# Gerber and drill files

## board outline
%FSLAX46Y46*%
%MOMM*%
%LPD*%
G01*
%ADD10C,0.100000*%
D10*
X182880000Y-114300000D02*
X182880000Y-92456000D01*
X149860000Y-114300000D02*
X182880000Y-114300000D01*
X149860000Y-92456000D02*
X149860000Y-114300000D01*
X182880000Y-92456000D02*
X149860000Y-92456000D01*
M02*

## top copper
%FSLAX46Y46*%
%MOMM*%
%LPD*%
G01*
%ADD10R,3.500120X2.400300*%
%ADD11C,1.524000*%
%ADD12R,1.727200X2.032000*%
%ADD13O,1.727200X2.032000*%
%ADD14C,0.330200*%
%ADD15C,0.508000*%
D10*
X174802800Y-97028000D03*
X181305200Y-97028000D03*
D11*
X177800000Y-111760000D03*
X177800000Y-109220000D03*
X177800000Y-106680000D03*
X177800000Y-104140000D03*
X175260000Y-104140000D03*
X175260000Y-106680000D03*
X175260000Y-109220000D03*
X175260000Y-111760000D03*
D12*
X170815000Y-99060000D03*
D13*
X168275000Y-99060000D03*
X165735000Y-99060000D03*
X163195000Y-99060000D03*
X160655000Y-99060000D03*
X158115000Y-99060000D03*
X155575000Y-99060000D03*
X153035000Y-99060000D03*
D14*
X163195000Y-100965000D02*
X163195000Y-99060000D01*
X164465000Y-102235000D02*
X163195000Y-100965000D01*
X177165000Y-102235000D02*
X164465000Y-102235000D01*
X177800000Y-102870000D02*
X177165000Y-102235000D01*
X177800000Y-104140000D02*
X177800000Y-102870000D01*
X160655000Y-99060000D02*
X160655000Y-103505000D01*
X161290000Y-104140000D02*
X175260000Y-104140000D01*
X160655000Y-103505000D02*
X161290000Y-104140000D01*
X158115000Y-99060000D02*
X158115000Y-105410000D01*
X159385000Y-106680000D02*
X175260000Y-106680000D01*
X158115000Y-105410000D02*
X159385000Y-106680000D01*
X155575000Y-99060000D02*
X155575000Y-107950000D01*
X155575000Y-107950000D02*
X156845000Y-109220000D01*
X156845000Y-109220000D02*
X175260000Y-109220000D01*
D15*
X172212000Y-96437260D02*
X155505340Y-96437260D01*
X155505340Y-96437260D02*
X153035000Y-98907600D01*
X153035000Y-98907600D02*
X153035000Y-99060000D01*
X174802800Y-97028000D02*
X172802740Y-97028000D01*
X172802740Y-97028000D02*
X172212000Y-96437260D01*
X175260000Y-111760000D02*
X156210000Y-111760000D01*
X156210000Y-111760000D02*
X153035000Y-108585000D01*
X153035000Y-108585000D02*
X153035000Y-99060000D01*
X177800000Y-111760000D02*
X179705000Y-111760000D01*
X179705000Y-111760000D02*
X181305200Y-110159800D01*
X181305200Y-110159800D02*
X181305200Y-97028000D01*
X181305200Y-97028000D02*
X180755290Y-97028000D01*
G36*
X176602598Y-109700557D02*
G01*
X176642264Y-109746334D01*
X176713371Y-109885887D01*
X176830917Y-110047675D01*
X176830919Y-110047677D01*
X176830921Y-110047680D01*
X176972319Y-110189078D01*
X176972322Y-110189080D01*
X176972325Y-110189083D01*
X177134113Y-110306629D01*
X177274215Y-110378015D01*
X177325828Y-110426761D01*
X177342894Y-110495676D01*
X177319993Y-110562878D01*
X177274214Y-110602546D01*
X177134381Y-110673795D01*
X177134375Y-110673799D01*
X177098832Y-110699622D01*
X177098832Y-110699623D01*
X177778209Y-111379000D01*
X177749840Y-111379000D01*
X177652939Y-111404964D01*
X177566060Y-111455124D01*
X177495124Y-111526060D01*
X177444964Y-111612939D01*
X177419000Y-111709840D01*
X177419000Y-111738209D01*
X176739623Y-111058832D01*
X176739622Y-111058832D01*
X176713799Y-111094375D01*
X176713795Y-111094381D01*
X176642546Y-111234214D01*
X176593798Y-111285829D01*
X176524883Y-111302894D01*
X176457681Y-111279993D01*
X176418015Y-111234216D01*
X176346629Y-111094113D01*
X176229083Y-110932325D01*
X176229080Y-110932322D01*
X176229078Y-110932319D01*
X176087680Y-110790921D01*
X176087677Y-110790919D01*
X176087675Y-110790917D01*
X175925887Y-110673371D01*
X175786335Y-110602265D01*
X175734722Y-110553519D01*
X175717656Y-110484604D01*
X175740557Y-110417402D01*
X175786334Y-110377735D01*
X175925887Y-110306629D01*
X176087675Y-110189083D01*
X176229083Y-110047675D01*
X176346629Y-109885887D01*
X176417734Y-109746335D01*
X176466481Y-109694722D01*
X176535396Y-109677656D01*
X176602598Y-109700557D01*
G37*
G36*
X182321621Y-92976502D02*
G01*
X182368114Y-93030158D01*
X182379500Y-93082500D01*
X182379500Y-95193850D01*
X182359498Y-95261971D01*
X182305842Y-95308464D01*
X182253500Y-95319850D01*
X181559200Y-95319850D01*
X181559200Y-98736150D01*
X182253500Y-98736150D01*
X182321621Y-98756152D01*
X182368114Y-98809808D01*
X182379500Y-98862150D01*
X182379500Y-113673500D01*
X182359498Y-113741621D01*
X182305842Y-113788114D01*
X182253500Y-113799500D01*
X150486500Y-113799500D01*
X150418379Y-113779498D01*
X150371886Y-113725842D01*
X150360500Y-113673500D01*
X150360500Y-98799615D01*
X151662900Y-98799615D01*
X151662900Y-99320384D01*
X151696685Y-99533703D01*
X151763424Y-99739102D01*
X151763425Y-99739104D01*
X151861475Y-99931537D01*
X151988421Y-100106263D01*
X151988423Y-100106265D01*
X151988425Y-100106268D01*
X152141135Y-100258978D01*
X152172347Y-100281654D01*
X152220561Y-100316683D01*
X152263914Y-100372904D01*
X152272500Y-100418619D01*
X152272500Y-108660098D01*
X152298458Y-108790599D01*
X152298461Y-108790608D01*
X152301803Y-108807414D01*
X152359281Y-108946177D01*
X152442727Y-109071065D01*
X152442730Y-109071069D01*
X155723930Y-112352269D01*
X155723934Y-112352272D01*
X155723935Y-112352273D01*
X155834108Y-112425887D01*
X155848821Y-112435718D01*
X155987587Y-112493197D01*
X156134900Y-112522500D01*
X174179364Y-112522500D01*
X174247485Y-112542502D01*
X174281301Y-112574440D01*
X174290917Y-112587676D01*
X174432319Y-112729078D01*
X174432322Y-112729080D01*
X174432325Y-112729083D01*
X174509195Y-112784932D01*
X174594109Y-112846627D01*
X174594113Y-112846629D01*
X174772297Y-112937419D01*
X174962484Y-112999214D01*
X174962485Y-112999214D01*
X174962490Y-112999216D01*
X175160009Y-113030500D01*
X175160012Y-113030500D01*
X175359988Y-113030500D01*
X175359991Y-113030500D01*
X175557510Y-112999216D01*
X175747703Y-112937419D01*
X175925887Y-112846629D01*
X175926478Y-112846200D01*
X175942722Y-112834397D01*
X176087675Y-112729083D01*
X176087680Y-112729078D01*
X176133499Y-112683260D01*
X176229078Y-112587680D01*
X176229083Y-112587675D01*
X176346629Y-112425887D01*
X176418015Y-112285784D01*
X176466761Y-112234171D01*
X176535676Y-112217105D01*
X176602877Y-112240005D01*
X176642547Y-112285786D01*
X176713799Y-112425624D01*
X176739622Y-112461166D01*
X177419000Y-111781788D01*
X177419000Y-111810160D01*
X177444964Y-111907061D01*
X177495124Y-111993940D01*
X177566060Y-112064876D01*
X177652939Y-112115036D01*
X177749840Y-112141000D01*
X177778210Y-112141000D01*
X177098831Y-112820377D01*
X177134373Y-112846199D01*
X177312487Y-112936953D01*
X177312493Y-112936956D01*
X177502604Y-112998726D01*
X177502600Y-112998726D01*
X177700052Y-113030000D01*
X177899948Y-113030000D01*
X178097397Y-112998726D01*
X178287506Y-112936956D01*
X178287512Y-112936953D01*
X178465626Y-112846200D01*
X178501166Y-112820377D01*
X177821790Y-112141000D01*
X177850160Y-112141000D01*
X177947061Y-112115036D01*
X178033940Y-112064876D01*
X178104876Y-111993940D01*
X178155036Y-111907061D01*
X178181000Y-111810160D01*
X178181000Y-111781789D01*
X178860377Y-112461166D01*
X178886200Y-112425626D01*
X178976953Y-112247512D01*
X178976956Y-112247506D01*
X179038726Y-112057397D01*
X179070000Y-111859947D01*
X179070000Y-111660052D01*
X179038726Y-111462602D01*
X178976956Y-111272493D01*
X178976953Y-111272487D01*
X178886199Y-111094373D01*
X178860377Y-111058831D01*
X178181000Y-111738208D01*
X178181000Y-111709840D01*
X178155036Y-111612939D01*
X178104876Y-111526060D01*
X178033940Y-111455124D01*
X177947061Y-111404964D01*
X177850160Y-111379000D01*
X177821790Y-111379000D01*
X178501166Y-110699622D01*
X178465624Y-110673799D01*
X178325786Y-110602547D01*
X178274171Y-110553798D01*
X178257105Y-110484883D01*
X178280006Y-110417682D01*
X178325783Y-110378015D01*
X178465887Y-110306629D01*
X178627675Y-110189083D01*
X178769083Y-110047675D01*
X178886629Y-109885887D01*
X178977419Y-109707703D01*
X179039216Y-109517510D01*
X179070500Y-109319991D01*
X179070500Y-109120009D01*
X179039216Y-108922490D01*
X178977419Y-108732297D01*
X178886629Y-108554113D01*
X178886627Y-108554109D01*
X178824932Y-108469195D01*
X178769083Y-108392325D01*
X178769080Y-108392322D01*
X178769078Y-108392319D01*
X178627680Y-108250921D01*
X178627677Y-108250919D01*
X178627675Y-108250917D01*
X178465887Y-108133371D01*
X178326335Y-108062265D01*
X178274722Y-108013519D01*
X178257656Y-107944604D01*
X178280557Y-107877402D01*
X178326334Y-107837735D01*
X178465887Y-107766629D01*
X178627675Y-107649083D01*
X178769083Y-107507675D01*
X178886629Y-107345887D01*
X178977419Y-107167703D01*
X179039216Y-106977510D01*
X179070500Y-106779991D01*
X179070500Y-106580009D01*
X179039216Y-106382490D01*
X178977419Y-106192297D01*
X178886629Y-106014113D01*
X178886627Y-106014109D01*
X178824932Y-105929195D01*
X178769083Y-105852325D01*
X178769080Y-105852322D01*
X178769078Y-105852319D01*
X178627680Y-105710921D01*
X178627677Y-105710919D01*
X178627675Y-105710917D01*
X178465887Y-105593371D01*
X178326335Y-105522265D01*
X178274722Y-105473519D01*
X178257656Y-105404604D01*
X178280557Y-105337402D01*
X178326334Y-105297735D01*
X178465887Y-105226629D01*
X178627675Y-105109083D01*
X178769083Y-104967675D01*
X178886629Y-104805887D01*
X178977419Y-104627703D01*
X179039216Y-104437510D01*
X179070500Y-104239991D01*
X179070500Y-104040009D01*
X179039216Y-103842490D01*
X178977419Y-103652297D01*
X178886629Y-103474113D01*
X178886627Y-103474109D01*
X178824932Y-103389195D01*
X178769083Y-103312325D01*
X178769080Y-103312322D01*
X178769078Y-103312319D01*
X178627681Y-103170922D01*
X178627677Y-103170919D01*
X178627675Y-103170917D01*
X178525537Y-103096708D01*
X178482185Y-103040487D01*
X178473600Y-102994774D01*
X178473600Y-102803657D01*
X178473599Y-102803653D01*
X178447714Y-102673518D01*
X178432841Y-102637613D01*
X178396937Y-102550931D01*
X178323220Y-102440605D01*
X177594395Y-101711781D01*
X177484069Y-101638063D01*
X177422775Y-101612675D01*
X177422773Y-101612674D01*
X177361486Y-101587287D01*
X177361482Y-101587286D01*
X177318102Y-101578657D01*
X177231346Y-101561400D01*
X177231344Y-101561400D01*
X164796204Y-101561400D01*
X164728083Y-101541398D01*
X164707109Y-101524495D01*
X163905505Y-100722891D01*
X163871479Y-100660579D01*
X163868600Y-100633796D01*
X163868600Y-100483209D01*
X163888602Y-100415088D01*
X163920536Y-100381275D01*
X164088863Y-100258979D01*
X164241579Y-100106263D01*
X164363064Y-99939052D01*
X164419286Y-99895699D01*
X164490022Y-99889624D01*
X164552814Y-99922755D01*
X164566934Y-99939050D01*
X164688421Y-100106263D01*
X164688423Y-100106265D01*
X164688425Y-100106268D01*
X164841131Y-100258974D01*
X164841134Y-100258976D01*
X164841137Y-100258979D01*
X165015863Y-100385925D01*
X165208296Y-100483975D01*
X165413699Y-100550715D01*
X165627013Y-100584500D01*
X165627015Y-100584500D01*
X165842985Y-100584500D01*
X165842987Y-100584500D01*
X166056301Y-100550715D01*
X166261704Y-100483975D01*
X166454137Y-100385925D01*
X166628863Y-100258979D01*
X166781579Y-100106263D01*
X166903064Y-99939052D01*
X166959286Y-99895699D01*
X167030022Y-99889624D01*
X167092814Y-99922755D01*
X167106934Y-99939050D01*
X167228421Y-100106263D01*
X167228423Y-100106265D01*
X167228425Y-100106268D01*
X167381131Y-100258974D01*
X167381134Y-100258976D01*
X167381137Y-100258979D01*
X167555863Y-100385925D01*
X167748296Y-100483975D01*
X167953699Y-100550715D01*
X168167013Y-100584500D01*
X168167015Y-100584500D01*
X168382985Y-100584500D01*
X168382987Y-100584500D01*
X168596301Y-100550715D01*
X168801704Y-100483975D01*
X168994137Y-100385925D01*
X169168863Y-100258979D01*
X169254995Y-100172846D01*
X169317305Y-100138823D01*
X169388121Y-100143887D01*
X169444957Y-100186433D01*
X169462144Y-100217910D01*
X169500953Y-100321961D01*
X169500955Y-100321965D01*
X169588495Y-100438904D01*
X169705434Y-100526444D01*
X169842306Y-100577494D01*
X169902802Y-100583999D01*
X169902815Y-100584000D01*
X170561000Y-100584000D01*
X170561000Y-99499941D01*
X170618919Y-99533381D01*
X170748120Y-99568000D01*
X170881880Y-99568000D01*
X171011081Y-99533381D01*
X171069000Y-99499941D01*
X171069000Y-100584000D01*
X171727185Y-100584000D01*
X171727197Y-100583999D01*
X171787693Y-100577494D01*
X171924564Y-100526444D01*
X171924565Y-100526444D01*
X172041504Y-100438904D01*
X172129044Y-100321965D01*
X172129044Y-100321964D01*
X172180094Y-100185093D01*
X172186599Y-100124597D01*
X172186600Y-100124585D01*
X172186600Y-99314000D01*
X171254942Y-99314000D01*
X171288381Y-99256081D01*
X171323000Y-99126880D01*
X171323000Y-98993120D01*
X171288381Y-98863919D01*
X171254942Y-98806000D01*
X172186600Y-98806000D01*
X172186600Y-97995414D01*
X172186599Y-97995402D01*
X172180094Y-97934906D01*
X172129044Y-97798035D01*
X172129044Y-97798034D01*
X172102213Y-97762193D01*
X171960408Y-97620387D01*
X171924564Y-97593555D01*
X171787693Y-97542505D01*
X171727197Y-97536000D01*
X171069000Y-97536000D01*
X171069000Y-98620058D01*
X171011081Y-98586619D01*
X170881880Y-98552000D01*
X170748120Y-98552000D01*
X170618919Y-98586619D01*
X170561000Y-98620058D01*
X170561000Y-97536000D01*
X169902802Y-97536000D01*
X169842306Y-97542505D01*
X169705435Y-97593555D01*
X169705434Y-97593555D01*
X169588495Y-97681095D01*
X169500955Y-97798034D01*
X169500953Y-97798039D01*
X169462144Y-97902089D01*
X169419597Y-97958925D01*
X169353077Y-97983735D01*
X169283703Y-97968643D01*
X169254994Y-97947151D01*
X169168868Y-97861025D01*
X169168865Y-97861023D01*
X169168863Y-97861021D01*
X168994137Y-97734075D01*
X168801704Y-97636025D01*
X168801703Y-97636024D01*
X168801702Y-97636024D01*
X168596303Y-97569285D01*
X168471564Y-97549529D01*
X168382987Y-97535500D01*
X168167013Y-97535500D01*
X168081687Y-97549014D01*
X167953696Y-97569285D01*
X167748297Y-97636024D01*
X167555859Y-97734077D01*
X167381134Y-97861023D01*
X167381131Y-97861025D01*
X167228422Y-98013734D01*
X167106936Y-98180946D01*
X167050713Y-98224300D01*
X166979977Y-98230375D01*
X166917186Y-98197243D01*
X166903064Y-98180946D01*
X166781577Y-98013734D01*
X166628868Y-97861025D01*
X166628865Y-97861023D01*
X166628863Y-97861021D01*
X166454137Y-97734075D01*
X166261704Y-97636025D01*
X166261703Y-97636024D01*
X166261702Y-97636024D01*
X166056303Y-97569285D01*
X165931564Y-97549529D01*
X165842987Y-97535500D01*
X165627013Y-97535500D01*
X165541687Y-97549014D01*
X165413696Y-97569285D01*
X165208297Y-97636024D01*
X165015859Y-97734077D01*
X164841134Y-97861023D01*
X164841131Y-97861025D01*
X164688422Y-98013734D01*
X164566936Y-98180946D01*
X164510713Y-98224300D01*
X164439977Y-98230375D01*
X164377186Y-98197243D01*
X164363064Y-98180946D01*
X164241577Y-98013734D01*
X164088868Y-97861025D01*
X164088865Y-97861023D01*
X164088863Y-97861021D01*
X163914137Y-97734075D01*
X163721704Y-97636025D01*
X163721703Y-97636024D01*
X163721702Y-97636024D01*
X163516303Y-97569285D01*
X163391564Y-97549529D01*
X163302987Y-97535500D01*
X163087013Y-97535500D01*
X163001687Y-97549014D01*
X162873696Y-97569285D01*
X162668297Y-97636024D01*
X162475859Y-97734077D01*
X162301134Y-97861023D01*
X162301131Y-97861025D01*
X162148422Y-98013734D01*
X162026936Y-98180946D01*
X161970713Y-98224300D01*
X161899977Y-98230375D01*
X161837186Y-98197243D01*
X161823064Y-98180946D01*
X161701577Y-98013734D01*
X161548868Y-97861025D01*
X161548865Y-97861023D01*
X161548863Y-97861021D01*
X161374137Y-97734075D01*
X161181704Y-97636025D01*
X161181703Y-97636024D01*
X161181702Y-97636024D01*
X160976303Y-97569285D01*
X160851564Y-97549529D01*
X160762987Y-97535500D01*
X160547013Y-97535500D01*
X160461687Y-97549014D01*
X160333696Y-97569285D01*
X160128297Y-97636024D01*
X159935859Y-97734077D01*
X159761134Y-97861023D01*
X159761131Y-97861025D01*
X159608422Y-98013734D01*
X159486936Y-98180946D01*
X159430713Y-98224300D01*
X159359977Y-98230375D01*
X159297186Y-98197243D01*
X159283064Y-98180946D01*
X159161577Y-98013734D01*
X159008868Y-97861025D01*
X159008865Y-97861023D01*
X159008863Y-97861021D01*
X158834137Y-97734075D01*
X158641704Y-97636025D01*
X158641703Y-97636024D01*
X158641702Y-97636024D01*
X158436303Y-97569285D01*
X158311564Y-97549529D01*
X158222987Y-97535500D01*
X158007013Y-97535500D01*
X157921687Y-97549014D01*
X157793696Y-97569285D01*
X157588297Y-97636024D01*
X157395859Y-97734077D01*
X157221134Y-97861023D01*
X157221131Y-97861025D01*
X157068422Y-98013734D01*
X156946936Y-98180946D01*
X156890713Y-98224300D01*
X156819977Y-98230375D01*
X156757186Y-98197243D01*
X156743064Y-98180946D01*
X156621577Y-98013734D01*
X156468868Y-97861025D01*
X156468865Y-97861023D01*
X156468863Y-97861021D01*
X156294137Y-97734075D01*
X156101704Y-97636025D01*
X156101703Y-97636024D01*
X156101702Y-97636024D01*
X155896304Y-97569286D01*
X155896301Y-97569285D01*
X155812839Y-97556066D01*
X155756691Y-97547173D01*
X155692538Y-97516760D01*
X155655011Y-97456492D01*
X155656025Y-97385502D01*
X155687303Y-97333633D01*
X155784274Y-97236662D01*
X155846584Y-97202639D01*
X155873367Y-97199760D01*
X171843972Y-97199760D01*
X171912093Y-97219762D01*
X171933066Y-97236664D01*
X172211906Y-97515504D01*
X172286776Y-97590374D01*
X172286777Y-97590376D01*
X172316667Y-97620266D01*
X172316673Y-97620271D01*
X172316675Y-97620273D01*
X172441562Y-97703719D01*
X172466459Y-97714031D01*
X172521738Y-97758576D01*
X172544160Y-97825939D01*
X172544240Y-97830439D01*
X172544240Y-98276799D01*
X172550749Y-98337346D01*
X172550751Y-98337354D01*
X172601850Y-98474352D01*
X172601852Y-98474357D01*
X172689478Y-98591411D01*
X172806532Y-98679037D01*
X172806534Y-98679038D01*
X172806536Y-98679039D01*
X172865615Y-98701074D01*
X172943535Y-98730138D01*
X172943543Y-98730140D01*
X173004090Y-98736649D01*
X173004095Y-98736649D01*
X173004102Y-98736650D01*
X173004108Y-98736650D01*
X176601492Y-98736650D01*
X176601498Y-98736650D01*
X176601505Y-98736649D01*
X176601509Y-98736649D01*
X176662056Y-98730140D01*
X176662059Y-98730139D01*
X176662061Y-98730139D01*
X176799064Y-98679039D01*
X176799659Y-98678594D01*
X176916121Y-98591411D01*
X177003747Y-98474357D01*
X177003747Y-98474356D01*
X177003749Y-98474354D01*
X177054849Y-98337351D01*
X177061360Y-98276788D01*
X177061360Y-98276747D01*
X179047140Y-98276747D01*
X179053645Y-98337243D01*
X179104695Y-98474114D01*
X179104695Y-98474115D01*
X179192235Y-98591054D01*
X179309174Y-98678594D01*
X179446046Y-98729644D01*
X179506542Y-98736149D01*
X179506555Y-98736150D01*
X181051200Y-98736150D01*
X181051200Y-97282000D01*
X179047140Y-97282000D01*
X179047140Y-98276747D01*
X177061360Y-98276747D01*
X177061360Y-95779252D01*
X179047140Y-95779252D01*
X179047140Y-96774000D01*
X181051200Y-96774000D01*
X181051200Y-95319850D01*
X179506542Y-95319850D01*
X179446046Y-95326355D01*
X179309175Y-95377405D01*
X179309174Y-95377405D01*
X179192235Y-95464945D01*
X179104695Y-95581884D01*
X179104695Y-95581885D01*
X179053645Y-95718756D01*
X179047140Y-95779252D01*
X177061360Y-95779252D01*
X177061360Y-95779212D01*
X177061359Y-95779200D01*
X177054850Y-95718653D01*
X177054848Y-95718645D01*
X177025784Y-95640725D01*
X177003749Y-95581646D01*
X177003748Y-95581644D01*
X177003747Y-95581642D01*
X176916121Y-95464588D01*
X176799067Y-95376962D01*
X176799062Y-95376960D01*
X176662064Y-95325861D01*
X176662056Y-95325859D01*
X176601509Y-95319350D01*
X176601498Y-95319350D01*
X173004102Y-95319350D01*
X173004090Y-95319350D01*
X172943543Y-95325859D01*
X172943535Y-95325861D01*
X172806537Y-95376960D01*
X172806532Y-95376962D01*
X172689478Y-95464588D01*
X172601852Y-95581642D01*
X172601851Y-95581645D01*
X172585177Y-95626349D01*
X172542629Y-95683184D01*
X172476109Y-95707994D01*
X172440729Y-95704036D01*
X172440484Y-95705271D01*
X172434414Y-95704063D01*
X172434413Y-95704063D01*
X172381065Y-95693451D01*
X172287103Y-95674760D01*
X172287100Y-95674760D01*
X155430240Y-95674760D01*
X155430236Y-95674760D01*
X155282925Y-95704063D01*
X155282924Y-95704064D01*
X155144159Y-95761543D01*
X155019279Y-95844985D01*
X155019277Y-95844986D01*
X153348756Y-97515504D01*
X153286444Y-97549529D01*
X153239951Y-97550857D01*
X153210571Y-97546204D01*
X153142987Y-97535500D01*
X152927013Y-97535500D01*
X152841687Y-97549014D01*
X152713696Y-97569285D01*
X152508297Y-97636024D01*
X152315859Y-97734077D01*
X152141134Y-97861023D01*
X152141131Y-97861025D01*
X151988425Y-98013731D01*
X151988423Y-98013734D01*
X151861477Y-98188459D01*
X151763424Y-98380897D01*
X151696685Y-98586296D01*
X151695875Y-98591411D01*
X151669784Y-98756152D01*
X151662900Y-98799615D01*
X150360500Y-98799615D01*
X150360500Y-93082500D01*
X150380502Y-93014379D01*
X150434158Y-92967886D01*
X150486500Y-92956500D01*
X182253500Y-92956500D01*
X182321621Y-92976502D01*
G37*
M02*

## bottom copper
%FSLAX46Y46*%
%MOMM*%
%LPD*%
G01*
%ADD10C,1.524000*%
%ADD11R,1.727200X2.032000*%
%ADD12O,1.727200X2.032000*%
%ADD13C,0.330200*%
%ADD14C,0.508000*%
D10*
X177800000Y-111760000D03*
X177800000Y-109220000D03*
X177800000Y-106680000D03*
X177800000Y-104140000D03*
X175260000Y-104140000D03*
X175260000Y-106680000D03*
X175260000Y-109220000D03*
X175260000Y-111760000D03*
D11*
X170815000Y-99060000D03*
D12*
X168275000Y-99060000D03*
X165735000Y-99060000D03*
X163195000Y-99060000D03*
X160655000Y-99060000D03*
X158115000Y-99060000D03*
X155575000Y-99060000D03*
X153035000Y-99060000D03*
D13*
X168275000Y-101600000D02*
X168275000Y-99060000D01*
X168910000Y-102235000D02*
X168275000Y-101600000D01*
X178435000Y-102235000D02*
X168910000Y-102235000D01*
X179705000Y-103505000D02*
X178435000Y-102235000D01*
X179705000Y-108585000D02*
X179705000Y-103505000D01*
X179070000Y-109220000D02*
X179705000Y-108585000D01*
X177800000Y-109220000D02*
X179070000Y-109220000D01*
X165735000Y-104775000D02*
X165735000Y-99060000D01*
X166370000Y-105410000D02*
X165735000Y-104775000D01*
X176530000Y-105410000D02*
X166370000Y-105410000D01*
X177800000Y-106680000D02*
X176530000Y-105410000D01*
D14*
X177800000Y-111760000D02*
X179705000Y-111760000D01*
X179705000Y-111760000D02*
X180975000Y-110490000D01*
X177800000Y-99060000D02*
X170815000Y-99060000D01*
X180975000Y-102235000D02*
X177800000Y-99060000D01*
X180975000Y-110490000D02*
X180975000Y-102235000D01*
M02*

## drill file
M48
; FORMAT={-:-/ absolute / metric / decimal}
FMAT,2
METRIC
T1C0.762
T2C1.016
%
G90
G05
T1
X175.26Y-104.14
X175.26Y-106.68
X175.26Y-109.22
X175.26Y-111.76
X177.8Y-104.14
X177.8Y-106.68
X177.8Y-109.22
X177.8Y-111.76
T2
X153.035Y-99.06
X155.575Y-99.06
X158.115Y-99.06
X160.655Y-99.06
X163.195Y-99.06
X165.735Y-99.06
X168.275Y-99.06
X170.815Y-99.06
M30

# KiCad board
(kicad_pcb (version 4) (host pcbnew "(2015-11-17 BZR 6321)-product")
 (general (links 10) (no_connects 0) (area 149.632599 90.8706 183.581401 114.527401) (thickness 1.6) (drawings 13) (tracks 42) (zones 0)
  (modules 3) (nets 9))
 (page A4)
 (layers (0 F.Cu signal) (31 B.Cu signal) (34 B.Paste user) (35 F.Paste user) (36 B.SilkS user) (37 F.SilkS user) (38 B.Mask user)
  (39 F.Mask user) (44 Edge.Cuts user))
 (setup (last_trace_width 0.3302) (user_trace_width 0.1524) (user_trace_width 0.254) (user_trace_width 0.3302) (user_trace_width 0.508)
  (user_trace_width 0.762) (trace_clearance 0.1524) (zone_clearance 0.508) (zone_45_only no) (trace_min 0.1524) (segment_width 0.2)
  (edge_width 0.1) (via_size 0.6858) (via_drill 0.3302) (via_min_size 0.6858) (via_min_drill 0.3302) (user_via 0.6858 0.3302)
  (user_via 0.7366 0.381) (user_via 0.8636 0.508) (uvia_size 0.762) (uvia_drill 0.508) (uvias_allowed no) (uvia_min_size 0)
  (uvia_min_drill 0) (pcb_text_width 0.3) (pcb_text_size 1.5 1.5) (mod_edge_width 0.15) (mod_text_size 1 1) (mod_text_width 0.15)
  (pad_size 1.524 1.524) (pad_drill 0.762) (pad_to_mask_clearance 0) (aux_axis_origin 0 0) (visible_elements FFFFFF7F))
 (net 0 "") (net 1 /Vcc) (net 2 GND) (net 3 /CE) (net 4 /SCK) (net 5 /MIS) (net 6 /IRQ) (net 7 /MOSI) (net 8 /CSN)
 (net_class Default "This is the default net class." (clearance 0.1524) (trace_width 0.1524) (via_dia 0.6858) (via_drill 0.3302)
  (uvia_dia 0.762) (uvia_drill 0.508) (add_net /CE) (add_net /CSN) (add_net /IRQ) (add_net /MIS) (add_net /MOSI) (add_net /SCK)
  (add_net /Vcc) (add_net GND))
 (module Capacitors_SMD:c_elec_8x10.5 (layer F.Cu) (at 178.054 97.028 180)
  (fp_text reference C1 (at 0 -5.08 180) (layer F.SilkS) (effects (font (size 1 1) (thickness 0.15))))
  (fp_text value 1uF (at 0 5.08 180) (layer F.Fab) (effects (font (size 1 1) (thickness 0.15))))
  (pad 1 smd rect (at 3.2512 0 180) (size 3.50012 2.4003) (layers F.Cu F.Paste F.Mask) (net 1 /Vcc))
  (pad 2 smd rect (at -3.2512 0 180) (size 3.50012 2.4003) (layers F.Cu F.Paste F.Mask) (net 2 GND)))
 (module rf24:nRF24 (layer F.Cu) (at 170.18 109.22)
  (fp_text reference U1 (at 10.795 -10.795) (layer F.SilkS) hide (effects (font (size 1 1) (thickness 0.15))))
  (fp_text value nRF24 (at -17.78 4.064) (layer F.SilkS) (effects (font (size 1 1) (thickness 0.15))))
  (pad 0 thru_hole circle (at 7.62 2.54) (size 1.524 1.524) (drill 0.762) (layers *.Cu *.Mask F.SilkS) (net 2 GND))
  (pad 1 thru_hole circle (at 7.62 0) (size 1.524 1.524) (drill 0.762) (layers *.Cu *.Mask F.SilkS) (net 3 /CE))
  (pad 2 thru_hole circle (at 7.62 -2.54) (size 1.524 1.524) (drill 0.762) (layers *.Cu *.Mask F.SilkS) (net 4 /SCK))
  (pad 3 thru_hole circle (at 7.62 -5.08) (size 1.524 1.524) (drill 0.762) (layers *.Cu *.Mask F.SilkS) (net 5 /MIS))
  (pad 4 thru_hole circle (at 5.08 -5.08) (size 1.524 1.524) (drill 0.762) (layers *.Cu *.Mask F.SilkS) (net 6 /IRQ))
  (pad 5 thru_hole circle (at 5.08 -2.54) (size 1.524 1.524) (drill 0.762) (layers *.Cu *.Mask F.SilkS) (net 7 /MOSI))
  (pad 6 thru_hole circle (at 5.08 0) (size 1.524 1.524) (drill 0.762) (layers *.Cu *.Mask F.SilkS) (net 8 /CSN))
  (pad 7 thru_hole circle (at 5.08 2.54) (size 1.524 1.524) (drill 0.762) (layers *.Cu *.Mask F.SilkS) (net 1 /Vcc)))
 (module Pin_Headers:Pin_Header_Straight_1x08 (layer F.Cu) (at 170.815 99.06 270)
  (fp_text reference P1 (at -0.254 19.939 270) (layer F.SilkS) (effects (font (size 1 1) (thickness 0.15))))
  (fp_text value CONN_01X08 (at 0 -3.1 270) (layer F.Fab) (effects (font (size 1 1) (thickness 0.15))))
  (pad 1 thru_hole rect (at 0 0 270) (size 2.032 1.7272) (drill 1.016) (layers *.Cu *.Mask F.SilkS) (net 2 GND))
  (pad 2 thru_hole oval (at 0 2.54 270) (size 2.032 1.7272) (drill 1.016) (layers *.Cu *.Mask F.SilkS) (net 3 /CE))
  (pad 3 thru_hole oval (at 0 5.08 270) (size 2.032 1.7272) (drill 1.016) (layers *.Cu *.Mask F.SilkS) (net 4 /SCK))
  (pad 4 thru_hole oval (at 0 7.62 270) (size 2.032 1.7272) (drill 1.016) (layers *.Cu *.Mask F.SilkS) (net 5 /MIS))
  (pad 5 thru_hole oval (at 0 10.16 270) (size 2.032 1.7272) (drill 1.016) (layers *.Cu *.Mask F.SilkS) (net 6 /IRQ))
  (pad 6 thru_hole oval (at 0 12.7 270) (size 2.032 1.7272) (drill 1.016) (layers *.Cu *.Mask F.SilkS) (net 7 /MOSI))
  (pad 7 thru_hole oval (at 0 15.24 270) (size 2.032 1.7272) (drill 1.016) (layers *.Cu *.Mask F.SilkS) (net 8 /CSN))
  (pad 8 thru_hole oval (at 0 17.78 270) (size 2.032 1.7272) (drill 1.016) (layers *.Cu *.Mask F.SilkS) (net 1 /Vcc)))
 (gr_line (start 182.88 114.3) (end 182.88 92.456) (angle 90) (layer Edge.Cuts) (width 0.1))
 (gr_line (start 149.86 114.3) (end 182.88 114.3) (angle 90) (layer Edge.Cuts) (width 0.1))
 (gr_line (start 149.86 92.456) (end 149.86 114.3) (angle 90) (layer Edge.Cuts) (width 0.1))
 (gr_line (start 182.88 92.456) (end 149.86 92.456) (angle 90) (layer Edge.Cuts) (width 0.1))
 (segment (start 168.275 101.6) (end 168.275 99.06) (width 0.3302) (layer B.Cu) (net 3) (status 20))
 (segment (start 168.91 102.235) (end 168.275 101.6) (width 0.3302) (layer B.Cu) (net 3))
 (segment (start 178.435 102.235) (end 168.91 102.235) (width 0.3302) (layer B.Cu) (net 3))
 (segment (start 179.705 103.505) (end 178.435 102.235) (width 0.3302) (layer B.Cu) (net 3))
 (segment (start 179.705 108.585) (end 179.705 103.505) (width 0.3302) (layer B.Cu) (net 3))
 (segment (start 179.07 109.22) (end 179.705 108.585) (width 0.3302) (layer B.Cu) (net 3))
 (segment (start 177.8 109.22) (end 179.07 109.22) (width 0.3302) (layer B.Cu) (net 3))
 (segment (start 165.735 104.775) (end 165.735 99.06) (width 0.3302) (layer B.Cu) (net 4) (status 20))
 (segment (start 166.37 105.41) (end 165.735 104.775) (width 0.3302) (layer B.Cu) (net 4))
 (segment (start 176.53 105.41) (end 166.37 105.41) (width 0.3302) (layer B.Cu) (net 4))
 (segment (start 177.8 106.68) (end 176.53 105.41) (width 0.3302) (layer B.Cu) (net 4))
 (segment (start 163.195 100.965) (end 163.195 99.06) (width 0.3302) (layer F.Cu) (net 5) (status 20))
 (segment (start 164.465 102.235) (end 163.195 100.965) (width 0.3302) (layer F.Cu) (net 5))
 (segment (start 177.165 102.235) (end 164.465 102.235) (width 0.3302) (layer F.Cu) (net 5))
 (segment (start 177.8 102.87) (end 177.165 102.235) (width 0.3302) (layer F.Cu) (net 5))
 (segment (start 177.8 104.14) (end 177.8 102.87) (width 0.3302) (layer F.Cu) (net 5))
 (segment (start 160.655 99.06) (end 160.655 103.505) (width 0.3302) (layer F.Cu) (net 6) (status 10))
 (segment (start 161.29 104.14) (end 175.26 104.14) (width 0.3302) (layer F.Cu) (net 6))
 (segment (start 160.655 103.505) (end 161.29 104.14) (width 0.3302) (layer F.Cu) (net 6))
 (segment (start 158.115 99.06) (end 158.115 105.41) (width 0.3302) (layer F.Cu) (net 7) (status 10))
 (segment (start 159.385 106.68) (end 175.26 106.68) (width 0.3302) (layer F.Cu) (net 7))
 (segment (start 158.115 105.41) (end 159.385 106.68) (width 0.3302) (layer F.Cu) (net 7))
 (segment (start 155.575 99.06) (end 155.575 107.95) (width 0.3302) (layer F.Cu) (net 8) (status 10))
 (segment (start 155.575 107.95) (end 156.845 109.22) (width 0.3302) (layer F.Cu) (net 8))
 (segment (start 156.845 109.22) (end 175.26 109.22) (width 0.3302) (layer F.Cu) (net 8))
 (segment (start 172.212 96.43726) (end 155.50534 96.43726) (width 0.508) (layer F.Cu) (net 1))
 (segment (start 155.50534 96.43726) (end 153.035 98.9076) (width 0.508) (layer F.Cu) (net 1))
 (segment (start 153.035 98.9076) (end 153.035 99.06) (width 0.508) (layer F.Cu) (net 1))
 (segment (start 174.8028 97.028) (end 172.80274 97.028) (width 0.508) (layer F.Cu) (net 1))
 (segment (start 172.80274 97.028) (end 172.212 96.43726) (width 0.508) (layer F.Cu) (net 1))
 (segment (start 175.26 111.76) (end 156.21 111.76) (width 0.508) (layer F.Cu) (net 1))
 (segment (start 156.21 111.76) (end 153.035 108.585) (width 0.508) (layer F.Cu) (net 1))
 (segment (start 153.035 108.585) (end 153.035 99.06) (width 0.508) (layer F.Cu) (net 1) (status 20))
 (segment (start 177.8 111.76) (end 179.705 111.76) (width 0.508) (layer F.Cu) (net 2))
 (segment (start 179.705 111.76) (end 181.3052 110.1598) (width 0.508) (layer F.Cu) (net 2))
 (segment (start 177.8 111.76) (end 179.705 111.76) (width 0.508) (layer B.Cu) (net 2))
 (segment (start 179.705 111.76) (end 180.975 110.49) (width 0.508) (layer B.Cu) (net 2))
 (segment (start 177.8 99.06) (end 170.815 99.06) (width 0.508) (layer B.Cu) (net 2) (status 20))
 (segment (start 180.975 102.235) (end 177.8 99.06) (width 0.508) (layer B.Cu) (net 2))
 (segment (start 180.975 110.49) (end 180.975 102.235) (width 0.508) (layer B.Cu) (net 2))
 (segment (start 181.3052 110.1598) (end 181.3052 97.028) (width 0.508) (layer F.Cu) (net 2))
 (segment (start 181.3052 97.028) (end 180.75529 97.028) (width 0.508) (layer F.Cu) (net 2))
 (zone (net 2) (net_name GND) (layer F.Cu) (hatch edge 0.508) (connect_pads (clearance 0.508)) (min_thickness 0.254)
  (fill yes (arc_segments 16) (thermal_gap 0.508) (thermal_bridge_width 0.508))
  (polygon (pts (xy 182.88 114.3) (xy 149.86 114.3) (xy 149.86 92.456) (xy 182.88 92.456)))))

